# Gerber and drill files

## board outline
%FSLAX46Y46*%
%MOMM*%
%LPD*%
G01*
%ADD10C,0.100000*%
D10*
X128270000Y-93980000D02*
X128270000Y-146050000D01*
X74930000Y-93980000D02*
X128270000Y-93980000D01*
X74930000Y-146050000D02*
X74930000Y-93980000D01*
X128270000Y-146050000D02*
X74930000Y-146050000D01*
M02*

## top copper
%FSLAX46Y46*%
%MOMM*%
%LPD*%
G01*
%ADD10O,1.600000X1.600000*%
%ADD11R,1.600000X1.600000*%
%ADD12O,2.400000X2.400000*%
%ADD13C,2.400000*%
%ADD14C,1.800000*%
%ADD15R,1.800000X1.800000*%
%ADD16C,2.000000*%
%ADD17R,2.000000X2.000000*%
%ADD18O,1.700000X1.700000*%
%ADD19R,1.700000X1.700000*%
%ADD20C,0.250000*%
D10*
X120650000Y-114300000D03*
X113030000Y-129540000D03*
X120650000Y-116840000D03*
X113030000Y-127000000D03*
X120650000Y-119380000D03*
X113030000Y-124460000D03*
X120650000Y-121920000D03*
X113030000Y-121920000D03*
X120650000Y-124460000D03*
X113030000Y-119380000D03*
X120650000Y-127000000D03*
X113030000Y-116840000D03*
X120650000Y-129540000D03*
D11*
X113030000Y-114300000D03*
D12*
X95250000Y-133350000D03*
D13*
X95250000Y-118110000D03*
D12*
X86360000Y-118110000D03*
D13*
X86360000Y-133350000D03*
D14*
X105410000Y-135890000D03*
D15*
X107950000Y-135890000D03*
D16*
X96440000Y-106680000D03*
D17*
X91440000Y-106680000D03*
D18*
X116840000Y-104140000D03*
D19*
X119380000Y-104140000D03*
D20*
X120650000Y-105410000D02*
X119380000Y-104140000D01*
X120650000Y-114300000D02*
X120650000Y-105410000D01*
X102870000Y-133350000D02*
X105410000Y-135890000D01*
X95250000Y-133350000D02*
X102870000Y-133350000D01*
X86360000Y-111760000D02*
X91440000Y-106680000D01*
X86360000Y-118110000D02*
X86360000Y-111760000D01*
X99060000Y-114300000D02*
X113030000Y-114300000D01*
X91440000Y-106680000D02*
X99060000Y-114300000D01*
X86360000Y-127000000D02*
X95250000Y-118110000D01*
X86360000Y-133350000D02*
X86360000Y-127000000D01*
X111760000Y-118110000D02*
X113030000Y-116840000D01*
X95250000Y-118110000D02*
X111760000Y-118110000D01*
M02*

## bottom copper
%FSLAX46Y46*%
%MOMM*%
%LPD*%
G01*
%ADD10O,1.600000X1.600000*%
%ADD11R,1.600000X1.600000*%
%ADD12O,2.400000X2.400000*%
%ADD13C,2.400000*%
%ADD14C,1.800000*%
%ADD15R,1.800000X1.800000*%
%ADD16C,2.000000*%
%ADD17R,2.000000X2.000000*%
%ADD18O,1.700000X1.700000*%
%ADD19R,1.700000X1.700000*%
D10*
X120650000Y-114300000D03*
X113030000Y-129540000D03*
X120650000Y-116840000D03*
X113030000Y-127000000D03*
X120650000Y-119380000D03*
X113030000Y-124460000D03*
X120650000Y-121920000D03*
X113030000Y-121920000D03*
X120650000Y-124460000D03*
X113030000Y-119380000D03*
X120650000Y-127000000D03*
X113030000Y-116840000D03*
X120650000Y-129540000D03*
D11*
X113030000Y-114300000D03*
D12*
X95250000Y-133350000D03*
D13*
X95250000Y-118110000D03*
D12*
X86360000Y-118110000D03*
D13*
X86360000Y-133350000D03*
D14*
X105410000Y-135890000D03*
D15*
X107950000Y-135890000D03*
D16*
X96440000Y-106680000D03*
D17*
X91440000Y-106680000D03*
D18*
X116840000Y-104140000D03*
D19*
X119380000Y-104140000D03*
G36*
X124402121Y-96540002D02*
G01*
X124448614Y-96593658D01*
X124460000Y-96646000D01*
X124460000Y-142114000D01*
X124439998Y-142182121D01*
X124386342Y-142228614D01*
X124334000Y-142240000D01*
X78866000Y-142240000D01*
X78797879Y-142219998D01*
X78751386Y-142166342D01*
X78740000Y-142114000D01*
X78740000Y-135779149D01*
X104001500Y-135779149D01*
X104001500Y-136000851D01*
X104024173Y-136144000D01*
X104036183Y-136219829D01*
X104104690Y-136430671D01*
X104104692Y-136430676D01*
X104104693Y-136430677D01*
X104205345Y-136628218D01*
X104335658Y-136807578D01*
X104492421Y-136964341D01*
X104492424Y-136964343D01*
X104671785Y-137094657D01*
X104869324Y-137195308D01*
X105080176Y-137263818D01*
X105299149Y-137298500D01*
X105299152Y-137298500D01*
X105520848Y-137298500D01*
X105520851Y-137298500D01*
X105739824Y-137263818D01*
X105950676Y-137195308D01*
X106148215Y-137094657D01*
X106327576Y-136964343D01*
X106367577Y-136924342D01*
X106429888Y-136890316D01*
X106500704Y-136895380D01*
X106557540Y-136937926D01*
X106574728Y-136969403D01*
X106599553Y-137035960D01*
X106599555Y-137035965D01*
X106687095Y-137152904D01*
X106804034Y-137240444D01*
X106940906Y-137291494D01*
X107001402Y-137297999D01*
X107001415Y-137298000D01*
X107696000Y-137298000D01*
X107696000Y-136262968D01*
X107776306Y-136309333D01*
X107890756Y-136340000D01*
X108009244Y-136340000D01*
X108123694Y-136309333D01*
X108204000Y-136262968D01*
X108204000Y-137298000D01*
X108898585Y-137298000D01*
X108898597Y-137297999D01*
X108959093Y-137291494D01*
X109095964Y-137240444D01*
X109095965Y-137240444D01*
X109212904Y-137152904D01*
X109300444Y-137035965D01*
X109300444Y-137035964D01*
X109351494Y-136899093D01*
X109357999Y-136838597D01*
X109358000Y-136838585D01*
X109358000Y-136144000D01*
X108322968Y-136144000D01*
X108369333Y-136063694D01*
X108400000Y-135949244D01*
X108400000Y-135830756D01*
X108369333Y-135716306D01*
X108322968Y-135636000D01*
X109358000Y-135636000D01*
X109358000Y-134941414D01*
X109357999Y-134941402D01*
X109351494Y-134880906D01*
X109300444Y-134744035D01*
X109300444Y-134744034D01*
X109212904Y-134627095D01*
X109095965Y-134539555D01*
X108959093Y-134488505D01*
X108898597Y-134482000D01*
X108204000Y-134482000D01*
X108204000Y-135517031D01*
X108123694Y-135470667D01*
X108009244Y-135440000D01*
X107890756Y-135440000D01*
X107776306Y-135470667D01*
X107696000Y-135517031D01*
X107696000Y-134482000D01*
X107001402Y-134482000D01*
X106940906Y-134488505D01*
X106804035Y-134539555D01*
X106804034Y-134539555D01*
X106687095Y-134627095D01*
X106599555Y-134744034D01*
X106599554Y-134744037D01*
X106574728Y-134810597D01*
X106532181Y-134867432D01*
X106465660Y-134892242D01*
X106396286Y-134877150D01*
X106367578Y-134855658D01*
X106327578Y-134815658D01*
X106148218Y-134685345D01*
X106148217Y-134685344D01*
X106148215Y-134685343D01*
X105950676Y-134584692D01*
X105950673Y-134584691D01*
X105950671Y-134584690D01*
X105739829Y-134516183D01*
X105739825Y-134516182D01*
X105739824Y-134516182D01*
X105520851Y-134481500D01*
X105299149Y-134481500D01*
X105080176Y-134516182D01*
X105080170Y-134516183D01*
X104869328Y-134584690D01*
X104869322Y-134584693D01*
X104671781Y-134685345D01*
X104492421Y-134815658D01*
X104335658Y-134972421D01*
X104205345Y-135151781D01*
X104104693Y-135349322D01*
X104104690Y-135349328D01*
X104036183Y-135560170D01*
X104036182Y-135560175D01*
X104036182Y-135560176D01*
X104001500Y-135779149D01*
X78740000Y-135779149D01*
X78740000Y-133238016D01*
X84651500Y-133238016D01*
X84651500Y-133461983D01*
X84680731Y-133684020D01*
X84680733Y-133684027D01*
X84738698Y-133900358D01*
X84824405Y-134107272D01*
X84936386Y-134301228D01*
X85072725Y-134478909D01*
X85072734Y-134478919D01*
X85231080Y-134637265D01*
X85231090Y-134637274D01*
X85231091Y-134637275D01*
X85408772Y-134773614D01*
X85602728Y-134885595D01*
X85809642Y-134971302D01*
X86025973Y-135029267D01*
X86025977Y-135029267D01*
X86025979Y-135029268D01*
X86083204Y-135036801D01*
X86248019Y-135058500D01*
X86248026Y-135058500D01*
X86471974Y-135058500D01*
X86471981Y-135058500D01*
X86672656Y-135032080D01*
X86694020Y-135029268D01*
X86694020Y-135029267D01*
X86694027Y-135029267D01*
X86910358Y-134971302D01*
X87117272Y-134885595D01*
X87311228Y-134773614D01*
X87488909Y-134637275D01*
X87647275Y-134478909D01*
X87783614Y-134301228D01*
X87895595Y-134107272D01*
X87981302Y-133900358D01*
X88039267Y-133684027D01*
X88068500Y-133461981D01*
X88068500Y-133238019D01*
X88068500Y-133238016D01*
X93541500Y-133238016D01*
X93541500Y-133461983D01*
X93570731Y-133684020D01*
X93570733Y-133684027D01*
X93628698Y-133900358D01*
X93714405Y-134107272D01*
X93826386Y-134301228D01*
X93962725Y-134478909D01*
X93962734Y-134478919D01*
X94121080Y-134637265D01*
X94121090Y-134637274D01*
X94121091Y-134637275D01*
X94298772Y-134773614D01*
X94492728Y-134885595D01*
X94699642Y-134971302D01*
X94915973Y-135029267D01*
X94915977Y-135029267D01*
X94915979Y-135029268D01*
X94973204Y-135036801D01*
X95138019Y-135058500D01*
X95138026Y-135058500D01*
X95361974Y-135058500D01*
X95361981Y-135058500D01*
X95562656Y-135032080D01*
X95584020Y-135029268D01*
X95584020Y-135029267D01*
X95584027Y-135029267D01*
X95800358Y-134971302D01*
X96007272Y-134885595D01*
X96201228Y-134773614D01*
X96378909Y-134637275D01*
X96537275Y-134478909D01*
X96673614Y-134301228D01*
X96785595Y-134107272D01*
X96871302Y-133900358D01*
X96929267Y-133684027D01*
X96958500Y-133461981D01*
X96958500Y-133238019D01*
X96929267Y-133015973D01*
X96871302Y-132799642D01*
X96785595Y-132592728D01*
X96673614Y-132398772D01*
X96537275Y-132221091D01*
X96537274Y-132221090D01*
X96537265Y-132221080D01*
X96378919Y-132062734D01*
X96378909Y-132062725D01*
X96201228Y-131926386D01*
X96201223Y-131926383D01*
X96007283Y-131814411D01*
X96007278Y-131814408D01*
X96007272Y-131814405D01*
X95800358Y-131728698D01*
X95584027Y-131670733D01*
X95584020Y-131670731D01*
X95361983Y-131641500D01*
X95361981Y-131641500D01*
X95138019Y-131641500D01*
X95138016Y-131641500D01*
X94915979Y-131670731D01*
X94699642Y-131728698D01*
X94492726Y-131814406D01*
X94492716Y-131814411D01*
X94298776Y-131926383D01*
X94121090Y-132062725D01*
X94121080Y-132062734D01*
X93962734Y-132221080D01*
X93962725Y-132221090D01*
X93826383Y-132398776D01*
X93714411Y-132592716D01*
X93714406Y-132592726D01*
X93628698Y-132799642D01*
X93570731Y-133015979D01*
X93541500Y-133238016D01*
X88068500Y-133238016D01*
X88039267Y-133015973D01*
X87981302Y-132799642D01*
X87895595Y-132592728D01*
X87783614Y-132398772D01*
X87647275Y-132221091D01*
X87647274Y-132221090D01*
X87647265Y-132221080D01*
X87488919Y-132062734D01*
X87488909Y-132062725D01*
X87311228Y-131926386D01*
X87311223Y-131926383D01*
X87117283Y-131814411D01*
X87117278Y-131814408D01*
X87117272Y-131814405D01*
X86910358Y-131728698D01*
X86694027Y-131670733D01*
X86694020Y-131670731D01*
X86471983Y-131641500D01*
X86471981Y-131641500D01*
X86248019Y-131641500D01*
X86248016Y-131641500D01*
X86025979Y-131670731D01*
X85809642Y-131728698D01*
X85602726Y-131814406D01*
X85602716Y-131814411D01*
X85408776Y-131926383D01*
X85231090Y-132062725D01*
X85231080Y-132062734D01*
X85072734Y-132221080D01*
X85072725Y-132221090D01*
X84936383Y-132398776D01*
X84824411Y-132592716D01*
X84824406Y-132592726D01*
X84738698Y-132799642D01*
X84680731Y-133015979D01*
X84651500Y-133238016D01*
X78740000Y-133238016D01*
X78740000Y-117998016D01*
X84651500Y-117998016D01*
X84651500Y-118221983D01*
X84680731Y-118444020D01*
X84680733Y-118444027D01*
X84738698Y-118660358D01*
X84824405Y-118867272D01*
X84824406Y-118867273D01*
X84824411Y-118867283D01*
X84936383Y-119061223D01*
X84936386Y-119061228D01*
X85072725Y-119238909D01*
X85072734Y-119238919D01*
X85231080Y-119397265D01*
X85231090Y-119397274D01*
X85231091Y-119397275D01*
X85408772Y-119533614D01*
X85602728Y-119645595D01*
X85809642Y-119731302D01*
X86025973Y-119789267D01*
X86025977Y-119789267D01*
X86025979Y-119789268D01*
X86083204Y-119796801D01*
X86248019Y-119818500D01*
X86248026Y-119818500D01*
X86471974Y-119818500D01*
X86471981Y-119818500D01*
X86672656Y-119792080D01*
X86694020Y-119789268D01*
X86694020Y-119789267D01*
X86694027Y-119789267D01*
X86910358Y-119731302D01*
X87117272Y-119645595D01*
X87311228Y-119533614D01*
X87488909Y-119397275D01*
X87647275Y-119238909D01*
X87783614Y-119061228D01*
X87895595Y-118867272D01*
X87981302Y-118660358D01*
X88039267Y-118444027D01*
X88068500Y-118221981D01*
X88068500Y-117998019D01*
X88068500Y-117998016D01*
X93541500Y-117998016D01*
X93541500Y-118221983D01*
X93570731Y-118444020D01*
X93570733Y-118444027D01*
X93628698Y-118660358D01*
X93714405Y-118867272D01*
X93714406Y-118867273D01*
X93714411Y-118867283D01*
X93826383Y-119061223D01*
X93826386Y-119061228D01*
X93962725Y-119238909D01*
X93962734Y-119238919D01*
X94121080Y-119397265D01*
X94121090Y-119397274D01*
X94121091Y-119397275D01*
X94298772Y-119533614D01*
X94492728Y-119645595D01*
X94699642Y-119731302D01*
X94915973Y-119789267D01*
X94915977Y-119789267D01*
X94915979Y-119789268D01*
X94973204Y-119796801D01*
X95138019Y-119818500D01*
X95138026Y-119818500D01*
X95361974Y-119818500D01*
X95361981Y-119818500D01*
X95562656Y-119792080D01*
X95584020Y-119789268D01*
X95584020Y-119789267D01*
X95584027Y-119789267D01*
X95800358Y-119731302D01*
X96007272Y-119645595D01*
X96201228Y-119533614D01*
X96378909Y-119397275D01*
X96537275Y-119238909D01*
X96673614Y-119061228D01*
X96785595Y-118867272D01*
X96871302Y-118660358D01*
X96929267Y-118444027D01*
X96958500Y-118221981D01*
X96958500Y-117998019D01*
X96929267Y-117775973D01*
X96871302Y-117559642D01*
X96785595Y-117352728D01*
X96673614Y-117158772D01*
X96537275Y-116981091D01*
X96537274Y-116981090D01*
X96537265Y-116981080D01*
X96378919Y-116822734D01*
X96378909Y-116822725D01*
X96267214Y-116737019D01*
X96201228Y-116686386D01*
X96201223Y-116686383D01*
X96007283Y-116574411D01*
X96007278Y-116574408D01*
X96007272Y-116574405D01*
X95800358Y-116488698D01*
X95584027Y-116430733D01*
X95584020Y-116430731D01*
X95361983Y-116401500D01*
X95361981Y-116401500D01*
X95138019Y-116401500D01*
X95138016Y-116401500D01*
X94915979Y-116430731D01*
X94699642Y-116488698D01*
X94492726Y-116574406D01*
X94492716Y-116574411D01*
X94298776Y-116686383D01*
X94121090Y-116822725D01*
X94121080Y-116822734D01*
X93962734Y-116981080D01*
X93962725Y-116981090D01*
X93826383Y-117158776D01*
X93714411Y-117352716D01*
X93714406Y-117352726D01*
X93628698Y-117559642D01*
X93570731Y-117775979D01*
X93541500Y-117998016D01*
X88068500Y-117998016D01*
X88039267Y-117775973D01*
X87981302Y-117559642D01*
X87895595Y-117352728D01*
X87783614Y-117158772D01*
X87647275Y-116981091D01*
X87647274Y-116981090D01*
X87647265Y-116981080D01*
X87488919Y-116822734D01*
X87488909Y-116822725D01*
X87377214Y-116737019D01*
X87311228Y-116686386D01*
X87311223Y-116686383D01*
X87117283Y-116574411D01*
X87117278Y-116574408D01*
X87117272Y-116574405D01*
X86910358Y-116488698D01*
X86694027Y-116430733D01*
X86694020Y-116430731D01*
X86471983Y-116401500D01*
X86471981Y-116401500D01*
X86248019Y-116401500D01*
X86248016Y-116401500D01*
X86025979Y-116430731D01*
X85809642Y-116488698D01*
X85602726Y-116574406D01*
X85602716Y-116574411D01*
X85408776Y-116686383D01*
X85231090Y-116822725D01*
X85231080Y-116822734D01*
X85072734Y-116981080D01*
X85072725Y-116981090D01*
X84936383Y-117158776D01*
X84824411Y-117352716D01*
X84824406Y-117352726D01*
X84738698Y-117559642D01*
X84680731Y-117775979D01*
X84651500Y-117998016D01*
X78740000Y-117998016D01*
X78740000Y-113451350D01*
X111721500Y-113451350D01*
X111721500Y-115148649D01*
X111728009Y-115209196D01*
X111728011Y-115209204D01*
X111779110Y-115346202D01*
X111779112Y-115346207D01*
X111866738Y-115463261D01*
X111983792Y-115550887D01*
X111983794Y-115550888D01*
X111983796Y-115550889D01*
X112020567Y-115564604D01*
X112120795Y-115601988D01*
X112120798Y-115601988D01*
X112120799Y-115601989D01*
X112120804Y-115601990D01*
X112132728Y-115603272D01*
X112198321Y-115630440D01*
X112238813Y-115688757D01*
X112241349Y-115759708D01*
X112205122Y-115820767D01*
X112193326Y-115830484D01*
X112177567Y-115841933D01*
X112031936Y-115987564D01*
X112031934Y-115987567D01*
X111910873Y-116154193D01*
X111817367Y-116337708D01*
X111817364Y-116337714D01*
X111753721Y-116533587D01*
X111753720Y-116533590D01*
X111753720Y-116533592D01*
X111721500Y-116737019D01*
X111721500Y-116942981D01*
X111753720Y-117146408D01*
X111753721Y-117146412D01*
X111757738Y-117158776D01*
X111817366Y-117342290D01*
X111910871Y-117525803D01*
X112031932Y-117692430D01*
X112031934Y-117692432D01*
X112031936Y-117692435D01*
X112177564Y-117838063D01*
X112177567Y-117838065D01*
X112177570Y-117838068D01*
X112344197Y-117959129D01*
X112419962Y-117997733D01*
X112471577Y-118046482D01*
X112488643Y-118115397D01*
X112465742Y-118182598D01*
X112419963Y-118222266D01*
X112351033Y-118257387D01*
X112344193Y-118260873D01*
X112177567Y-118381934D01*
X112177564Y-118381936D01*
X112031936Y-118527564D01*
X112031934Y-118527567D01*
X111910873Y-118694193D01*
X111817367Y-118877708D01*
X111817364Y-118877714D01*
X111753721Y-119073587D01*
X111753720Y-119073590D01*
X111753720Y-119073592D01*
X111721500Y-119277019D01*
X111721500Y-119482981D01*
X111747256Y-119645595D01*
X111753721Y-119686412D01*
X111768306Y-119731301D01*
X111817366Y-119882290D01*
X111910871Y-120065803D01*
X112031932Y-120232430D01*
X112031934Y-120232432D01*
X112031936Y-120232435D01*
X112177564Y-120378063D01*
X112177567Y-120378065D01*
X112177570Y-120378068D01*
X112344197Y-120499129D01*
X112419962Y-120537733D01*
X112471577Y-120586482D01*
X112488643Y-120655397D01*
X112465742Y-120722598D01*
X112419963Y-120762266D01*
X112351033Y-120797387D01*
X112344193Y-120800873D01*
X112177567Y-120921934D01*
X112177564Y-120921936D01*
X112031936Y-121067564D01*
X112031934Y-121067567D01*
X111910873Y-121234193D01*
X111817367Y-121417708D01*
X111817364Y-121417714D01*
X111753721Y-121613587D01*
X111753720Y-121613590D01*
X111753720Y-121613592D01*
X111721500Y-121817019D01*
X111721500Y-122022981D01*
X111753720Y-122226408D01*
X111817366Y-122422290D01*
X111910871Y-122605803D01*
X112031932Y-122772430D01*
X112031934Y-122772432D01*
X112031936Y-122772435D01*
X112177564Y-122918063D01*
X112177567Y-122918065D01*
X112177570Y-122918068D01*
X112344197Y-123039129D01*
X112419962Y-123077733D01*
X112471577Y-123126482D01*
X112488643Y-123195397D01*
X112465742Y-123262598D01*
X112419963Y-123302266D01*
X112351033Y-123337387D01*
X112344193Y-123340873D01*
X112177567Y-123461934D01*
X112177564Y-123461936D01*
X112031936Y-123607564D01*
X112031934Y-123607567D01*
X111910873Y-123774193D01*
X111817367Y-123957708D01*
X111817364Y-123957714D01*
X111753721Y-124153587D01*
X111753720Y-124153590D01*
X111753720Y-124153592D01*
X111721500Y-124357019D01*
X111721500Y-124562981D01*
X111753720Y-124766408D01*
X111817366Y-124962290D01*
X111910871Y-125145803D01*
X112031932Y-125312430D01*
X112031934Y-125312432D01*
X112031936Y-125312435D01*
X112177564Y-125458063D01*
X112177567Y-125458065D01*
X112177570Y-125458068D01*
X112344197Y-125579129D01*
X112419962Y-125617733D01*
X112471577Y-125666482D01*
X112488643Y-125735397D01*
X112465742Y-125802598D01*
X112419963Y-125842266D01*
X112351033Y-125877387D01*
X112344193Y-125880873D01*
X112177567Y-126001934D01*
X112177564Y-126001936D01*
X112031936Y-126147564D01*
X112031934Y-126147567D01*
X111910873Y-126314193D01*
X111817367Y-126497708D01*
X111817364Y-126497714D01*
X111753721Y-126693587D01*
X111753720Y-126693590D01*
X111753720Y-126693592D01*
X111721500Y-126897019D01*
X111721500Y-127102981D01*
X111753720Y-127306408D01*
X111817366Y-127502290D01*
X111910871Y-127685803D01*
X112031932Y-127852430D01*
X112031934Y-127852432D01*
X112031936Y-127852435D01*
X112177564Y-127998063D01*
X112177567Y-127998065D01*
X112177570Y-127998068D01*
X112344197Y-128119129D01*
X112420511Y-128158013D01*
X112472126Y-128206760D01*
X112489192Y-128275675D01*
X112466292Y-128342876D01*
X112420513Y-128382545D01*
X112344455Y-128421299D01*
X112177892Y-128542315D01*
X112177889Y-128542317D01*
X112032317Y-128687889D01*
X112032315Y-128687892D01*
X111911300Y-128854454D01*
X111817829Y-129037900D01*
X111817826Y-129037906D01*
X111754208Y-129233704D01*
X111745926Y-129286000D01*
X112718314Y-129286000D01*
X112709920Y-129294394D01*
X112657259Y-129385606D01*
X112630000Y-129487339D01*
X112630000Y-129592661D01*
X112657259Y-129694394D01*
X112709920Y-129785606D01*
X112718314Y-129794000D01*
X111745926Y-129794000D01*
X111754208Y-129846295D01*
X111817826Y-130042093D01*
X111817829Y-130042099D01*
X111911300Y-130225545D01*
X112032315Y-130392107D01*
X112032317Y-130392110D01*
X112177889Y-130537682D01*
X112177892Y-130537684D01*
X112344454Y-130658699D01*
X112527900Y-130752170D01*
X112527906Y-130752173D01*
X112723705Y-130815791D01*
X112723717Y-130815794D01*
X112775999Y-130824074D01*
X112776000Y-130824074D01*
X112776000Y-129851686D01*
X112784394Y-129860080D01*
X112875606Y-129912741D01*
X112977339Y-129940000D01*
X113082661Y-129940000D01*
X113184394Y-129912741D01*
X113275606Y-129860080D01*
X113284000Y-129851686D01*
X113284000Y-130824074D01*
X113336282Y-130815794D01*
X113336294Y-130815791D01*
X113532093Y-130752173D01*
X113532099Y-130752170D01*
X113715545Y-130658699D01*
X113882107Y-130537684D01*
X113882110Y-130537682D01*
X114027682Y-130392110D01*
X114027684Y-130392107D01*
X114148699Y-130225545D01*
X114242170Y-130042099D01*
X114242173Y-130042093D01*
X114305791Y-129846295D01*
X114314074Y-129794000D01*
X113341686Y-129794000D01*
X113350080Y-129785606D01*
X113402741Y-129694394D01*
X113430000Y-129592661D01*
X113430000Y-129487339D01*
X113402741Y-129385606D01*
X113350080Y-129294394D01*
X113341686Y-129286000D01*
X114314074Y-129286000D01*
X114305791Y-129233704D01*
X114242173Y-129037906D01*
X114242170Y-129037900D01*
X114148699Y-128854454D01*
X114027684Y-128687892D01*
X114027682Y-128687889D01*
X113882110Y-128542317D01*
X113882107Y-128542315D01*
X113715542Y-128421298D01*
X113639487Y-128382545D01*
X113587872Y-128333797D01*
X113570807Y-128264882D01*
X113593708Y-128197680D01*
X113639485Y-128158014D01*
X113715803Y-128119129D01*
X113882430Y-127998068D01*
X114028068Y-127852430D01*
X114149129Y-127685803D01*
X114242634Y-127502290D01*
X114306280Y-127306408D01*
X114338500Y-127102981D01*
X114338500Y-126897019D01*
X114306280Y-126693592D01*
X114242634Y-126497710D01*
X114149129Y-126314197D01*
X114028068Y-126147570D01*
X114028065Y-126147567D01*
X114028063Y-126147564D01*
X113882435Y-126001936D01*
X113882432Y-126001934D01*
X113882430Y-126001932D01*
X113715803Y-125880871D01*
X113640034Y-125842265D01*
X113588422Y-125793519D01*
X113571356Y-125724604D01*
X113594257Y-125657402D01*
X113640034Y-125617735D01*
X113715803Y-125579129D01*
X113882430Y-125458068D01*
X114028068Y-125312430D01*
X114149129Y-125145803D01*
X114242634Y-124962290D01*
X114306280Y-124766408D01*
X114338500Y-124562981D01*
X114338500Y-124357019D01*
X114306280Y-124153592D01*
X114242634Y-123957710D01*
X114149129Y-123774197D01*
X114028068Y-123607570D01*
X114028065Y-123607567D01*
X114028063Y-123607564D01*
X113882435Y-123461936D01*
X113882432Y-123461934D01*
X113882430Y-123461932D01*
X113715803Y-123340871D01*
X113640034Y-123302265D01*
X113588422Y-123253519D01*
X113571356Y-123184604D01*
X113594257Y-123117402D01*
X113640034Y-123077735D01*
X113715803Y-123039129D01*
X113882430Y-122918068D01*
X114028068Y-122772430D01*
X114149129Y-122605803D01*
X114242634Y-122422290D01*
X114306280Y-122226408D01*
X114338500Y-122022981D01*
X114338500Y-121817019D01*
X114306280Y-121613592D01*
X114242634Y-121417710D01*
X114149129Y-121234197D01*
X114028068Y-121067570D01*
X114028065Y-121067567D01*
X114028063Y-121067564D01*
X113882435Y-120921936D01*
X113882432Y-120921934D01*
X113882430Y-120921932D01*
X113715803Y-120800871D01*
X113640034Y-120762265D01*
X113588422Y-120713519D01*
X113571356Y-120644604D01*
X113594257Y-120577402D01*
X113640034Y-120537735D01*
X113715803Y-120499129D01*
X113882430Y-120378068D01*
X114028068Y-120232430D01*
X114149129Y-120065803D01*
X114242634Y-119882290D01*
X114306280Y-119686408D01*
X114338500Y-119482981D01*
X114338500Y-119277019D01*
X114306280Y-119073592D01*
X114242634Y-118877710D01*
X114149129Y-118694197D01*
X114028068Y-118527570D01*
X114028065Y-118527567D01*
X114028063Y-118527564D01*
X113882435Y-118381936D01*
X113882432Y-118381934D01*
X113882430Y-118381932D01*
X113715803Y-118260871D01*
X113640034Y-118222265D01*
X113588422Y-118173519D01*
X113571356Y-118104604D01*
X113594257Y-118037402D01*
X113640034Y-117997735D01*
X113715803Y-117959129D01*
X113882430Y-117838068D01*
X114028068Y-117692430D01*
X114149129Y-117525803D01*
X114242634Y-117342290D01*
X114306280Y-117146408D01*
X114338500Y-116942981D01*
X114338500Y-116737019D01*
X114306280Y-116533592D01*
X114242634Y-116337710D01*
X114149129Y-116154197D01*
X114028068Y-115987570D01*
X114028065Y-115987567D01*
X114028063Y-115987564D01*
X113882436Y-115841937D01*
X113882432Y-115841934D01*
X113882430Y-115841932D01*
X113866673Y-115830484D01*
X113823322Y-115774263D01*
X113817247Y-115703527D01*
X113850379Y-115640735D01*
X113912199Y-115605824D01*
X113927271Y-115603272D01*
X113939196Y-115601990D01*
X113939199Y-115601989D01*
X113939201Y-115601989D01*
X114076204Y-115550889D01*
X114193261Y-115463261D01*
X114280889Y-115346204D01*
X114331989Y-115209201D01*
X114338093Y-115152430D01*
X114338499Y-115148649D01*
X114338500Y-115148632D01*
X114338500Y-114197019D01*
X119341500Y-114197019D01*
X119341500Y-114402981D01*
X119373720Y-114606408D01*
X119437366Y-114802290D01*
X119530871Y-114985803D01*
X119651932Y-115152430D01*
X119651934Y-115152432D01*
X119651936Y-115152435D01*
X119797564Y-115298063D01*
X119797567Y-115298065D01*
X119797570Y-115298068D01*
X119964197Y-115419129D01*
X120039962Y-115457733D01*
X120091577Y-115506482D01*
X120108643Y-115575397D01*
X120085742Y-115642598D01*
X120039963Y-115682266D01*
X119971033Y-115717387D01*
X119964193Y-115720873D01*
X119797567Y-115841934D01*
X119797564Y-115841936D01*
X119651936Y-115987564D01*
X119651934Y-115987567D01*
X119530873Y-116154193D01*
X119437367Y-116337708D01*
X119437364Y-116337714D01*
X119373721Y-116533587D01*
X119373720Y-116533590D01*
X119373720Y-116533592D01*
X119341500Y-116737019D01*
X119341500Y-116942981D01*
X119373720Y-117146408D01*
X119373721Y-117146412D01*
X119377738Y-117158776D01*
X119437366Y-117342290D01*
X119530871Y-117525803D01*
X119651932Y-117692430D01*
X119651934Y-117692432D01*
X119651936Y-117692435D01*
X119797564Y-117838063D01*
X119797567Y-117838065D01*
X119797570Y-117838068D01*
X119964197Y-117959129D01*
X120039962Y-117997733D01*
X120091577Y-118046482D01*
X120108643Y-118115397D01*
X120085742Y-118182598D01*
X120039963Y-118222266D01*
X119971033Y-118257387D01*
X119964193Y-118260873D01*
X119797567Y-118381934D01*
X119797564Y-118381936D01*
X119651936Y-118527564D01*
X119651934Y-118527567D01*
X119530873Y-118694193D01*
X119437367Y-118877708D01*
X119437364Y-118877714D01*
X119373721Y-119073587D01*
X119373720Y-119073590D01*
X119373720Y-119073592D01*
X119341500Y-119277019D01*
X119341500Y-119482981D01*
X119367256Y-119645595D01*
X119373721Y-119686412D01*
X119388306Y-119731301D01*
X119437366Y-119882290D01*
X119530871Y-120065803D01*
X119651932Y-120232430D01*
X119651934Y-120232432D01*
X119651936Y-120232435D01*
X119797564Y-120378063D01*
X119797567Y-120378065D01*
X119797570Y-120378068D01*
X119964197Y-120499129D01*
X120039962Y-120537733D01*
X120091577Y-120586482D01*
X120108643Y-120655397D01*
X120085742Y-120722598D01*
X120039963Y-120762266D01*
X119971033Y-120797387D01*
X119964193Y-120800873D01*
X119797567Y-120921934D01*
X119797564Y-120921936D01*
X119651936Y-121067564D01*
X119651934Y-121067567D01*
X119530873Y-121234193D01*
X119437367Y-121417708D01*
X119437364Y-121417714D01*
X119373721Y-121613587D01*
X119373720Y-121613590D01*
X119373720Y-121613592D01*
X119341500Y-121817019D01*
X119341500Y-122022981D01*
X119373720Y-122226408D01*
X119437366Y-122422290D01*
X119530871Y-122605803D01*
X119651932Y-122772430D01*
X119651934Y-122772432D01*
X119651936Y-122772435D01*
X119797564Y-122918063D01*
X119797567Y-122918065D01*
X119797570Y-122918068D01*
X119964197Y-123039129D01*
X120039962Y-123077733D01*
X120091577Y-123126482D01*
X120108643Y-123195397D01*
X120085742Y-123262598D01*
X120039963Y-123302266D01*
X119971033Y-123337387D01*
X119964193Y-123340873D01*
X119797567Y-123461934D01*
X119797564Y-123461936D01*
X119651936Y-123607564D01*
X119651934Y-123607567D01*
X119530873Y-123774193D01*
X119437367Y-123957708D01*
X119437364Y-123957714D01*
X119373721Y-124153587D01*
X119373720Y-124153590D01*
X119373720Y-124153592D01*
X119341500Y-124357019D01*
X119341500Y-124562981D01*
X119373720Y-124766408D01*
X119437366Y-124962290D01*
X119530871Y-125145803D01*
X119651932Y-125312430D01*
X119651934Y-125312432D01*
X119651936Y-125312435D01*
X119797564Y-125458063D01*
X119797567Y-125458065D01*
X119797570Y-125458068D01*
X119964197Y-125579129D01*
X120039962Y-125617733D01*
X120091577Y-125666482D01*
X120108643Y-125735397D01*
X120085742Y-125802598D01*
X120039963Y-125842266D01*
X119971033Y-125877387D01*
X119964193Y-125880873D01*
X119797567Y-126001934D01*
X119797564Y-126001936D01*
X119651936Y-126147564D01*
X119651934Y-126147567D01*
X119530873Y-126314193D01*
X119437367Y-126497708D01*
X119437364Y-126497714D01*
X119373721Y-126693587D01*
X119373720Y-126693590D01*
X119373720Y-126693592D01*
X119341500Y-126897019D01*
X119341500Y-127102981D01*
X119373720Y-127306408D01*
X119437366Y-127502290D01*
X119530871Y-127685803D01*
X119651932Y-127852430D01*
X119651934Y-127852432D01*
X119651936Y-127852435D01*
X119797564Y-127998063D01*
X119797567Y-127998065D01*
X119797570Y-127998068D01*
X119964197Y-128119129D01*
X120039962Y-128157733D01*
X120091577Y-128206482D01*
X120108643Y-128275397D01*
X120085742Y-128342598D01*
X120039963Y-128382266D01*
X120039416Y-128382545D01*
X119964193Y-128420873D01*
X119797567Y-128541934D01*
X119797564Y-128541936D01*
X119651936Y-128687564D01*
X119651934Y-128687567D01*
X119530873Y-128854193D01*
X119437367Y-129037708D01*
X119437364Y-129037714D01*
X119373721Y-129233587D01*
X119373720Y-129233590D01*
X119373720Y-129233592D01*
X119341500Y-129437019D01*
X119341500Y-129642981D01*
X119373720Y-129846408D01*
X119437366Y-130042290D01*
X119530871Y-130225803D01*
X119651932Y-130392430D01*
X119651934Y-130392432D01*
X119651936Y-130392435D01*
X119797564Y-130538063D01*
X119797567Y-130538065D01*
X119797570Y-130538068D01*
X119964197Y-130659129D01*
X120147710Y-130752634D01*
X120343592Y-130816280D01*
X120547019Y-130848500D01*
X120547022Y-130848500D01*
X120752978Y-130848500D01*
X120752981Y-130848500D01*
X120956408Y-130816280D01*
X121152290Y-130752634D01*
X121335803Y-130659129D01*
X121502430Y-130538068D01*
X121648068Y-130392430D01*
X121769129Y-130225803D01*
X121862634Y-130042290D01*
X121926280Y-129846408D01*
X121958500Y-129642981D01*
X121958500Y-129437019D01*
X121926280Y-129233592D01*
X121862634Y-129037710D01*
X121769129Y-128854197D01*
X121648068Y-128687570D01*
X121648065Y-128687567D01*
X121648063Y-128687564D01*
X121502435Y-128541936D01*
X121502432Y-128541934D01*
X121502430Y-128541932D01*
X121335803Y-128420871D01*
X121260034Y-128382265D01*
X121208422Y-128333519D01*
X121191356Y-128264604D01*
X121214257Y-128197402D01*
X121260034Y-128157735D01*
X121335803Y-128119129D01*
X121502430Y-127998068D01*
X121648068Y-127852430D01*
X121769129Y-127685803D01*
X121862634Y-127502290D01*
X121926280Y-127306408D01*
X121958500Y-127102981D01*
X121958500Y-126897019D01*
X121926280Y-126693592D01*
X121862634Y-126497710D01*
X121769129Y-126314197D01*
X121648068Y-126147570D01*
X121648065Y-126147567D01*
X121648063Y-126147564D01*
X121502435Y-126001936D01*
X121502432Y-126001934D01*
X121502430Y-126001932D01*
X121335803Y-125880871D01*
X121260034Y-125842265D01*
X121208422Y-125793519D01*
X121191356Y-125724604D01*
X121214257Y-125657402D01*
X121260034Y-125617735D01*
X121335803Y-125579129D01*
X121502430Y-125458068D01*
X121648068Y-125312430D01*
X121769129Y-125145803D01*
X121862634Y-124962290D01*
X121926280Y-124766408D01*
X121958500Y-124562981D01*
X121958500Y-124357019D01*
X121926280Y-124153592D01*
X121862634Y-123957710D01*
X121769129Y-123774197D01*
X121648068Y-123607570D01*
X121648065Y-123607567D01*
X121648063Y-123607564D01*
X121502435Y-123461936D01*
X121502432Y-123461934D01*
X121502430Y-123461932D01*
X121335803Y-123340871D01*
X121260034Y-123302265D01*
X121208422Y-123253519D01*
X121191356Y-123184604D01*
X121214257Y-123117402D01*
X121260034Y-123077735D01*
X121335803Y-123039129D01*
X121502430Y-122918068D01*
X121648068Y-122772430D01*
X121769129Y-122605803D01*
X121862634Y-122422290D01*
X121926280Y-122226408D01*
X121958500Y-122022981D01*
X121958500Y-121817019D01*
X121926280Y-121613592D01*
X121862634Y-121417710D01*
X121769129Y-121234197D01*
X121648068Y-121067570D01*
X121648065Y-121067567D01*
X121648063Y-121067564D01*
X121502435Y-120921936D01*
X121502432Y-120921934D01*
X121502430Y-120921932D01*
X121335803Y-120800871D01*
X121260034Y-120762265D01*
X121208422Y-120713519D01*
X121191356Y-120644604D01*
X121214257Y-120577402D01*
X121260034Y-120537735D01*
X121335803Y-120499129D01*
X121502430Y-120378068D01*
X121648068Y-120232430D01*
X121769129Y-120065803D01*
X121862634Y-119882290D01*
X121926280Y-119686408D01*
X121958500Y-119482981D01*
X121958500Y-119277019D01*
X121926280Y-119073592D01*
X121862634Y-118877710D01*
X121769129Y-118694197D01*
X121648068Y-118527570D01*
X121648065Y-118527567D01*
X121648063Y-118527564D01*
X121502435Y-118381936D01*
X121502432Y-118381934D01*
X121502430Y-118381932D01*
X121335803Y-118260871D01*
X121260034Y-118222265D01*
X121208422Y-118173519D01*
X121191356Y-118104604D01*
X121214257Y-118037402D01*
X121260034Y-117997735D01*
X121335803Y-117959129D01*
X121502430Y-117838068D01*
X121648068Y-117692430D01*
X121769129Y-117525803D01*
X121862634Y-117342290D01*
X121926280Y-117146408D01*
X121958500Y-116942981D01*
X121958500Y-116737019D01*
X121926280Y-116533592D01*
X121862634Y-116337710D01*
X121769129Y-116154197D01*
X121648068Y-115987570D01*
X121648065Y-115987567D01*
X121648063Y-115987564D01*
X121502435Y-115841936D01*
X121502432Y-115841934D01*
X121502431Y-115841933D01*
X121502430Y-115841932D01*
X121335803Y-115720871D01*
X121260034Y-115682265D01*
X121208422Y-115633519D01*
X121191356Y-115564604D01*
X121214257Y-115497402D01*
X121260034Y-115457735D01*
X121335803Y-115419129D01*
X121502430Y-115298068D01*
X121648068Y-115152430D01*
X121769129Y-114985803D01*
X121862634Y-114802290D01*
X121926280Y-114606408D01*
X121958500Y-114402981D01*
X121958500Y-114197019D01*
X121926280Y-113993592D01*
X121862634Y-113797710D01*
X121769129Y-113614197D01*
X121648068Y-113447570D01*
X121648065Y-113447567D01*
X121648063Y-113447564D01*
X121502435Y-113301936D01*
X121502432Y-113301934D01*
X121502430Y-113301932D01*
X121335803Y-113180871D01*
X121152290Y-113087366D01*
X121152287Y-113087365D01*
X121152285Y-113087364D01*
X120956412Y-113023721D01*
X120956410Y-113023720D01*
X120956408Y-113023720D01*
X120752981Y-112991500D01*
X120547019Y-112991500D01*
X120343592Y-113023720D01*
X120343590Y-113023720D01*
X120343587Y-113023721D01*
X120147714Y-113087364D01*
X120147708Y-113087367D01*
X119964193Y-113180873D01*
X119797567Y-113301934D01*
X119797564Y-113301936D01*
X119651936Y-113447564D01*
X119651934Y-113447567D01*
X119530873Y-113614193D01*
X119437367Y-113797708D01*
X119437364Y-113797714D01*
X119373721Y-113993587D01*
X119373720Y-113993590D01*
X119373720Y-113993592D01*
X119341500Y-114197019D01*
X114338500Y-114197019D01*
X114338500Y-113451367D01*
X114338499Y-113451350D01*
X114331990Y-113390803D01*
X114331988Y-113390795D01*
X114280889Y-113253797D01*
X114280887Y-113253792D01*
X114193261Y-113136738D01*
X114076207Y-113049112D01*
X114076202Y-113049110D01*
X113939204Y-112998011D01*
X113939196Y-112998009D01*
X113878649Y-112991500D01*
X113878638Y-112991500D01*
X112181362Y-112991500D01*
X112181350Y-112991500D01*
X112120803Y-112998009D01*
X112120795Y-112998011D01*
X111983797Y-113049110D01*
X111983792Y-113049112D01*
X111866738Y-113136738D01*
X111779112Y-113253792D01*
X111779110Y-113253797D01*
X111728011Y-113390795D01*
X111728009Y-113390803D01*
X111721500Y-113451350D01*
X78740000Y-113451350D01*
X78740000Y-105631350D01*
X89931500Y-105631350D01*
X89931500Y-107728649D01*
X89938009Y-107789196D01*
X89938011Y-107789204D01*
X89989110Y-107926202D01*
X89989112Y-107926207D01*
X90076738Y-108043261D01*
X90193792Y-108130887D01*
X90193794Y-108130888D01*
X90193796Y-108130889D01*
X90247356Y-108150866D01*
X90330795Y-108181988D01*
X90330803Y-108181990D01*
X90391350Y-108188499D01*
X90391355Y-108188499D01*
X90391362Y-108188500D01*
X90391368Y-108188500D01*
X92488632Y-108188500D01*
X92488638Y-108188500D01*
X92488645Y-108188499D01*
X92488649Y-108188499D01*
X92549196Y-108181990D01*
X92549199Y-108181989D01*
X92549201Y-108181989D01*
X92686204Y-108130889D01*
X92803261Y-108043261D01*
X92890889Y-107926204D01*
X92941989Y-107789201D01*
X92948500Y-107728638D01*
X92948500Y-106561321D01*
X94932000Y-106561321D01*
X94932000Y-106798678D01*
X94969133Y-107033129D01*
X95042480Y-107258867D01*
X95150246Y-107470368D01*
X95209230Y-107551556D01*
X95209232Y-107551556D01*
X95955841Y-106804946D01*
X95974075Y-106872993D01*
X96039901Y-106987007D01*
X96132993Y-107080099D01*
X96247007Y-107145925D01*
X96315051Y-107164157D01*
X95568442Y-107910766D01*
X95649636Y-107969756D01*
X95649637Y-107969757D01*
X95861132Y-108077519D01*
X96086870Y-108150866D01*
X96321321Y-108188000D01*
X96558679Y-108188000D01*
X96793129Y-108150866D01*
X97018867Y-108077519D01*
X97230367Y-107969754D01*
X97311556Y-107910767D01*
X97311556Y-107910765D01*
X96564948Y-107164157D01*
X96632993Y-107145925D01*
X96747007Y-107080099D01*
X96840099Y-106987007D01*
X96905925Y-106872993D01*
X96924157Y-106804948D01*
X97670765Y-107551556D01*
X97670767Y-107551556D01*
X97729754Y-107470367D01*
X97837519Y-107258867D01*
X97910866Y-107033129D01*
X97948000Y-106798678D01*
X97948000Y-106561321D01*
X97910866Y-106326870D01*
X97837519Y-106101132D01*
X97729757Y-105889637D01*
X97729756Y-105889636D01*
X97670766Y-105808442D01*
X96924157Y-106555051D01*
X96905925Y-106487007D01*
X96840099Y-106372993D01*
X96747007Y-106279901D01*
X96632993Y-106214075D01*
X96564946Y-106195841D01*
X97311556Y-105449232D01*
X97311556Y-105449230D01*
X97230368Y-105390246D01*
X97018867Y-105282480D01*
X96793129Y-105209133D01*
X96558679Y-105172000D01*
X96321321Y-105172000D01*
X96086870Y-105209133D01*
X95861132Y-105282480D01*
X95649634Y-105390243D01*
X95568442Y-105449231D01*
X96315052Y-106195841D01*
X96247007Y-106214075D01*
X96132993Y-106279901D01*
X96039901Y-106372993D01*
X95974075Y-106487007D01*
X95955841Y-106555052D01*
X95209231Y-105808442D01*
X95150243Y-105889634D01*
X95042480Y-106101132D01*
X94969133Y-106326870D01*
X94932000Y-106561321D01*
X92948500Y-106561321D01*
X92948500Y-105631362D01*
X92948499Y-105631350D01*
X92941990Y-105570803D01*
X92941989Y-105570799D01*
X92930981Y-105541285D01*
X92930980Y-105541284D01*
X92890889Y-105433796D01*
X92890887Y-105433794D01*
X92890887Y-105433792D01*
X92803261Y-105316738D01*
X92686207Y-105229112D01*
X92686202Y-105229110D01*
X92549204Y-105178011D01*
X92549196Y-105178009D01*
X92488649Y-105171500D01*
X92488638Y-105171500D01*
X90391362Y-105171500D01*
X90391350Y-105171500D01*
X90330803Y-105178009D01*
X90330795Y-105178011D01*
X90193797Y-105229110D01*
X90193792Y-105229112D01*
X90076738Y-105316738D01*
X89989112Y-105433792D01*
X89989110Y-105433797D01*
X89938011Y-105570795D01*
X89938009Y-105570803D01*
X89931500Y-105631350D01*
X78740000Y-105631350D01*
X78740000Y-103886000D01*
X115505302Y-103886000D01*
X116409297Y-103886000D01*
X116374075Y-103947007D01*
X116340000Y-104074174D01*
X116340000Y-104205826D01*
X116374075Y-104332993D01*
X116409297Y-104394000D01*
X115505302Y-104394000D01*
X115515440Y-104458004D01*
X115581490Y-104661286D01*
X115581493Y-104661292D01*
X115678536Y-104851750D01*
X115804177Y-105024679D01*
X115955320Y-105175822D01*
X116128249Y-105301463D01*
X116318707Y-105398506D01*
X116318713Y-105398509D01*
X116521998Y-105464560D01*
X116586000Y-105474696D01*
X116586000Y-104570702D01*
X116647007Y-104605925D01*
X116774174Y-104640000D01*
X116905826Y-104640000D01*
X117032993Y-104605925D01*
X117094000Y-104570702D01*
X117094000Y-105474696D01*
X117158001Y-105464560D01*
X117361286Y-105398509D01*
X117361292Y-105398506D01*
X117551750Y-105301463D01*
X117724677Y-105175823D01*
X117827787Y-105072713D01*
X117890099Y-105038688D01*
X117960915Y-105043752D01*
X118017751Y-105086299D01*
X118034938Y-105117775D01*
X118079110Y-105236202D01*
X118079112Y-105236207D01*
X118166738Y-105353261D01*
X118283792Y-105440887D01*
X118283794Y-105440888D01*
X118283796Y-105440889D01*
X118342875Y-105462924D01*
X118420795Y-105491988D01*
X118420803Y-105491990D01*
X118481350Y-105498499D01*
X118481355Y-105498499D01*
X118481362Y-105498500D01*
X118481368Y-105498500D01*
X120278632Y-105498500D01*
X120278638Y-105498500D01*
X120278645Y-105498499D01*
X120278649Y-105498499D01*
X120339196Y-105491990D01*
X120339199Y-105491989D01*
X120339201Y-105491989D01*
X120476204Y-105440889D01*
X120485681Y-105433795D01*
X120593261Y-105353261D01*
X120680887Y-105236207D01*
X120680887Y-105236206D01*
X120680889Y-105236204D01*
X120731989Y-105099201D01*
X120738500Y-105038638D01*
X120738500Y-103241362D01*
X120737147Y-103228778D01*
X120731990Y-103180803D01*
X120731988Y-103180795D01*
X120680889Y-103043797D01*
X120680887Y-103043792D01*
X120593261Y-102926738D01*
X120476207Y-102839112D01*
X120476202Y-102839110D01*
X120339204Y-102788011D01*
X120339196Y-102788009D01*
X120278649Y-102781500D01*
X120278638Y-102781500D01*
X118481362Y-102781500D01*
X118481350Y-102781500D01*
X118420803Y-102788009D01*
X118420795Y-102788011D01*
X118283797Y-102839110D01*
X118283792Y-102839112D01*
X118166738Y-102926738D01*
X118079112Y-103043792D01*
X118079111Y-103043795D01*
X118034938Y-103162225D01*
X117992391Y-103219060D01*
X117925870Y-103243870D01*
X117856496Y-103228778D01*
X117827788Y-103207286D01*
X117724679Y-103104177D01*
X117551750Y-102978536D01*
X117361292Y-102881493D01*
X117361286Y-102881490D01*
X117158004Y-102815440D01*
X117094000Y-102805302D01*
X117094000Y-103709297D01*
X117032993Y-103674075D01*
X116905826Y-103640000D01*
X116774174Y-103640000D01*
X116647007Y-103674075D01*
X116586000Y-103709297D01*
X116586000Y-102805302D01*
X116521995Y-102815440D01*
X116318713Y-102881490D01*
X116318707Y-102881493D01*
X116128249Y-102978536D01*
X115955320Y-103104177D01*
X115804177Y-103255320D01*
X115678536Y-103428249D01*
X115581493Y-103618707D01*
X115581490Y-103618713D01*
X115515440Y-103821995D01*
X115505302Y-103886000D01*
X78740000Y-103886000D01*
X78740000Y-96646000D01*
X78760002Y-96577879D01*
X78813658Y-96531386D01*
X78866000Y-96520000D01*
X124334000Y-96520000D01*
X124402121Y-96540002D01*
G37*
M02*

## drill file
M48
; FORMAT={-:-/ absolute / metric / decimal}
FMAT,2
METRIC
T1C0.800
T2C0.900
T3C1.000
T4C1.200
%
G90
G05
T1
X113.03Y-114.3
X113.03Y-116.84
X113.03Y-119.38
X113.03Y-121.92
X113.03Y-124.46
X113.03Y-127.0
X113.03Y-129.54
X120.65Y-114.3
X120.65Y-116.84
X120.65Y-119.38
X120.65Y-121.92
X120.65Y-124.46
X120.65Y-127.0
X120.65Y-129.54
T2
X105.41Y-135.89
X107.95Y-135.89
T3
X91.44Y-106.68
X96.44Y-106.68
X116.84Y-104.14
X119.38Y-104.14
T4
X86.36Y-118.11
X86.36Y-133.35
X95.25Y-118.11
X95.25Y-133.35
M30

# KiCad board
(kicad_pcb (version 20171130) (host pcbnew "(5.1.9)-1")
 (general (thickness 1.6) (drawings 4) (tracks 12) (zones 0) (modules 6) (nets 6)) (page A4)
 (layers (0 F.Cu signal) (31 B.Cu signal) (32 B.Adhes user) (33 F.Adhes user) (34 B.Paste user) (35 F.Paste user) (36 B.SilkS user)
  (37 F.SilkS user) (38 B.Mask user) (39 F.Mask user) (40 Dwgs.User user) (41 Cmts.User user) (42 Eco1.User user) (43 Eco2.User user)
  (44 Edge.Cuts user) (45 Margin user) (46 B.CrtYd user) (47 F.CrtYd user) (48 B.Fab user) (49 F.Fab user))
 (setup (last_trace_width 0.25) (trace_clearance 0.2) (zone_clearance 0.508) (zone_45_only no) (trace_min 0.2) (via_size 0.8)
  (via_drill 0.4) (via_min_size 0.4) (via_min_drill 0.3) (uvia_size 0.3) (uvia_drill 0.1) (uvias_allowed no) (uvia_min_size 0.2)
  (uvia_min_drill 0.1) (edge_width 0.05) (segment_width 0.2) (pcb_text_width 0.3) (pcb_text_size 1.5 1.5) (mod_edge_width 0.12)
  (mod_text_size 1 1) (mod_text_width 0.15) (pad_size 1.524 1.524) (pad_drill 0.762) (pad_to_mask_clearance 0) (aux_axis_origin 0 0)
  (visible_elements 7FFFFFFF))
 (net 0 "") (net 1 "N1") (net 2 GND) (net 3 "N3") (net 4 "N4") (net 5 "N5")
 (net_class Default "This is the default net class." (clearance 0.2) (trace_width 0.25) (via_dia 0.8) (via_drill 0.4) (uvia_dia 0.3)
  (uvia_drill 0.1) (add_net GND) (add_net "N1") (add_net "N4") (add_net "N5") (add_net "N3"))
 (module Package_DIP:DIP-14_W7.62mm (layer F.Cu) (at 113.03 114.3)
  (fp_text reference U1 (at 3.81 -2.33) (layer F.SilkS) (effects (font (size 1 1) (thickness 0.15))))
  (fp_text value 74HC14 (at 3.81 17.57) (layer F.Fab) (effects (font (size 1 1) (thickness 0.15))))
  (pad 14 thru_hole oval (at 7.62 0) (size 1.6 1.6) (drill 0.8) (layers *.Cu *.Mask) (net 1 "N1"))
  (pad 7 thru_hole oval (at 0 15.24) (size 1.6 1.6) (drill 0.8) (layers *.Cu *.Mask) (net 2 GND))
  (pad 13 thru_hole oval (at 7.62 2.54) (size 1.6 1.6) (drill 0.8) (layers *.Cu *.Mask))
  (pad 6 thru_hole oval (at 0 12.7) (size 1.6 1.6) (drill 0.8) (layers *.Cu *.Mask))
  (pad 12 thru_hole oval (at 7.62 5.08) (size 1.6 1.6) (drill 0.8) (layers *.Cu *.Mask))
  (pad 5 thru_hole oval (at 0 10.16) (size 1.6 1.6) (drill 0.8) (layers *.Cu *.Mask))
  (pad 11 thru_hole oval (at 7.62 7.62) (size 1.6 1.6) (drill 0.8) (layers *.Cu *.Mask))
  (pad 4 thru_hole oval (at 0 7.62) (size 1.6 1.6) (drill 0.8) (layers *.Cu *.Mask))
  (pad 10 thru_hole oval (at 7.62 10.16) (size 1.6 1.6) (drill 0.8) (layers *.Cu *.Mask))
  (pad 3 thru_hole oval (at 0 5.08) (size 1.6 1.6) (drill 0.8) (layers *.Cu *.Mask))
  (pad 9 thru_hole oval (at 7.62 12.7) (size 1.6 1.6) (drill 0.8) (layers *.Cu *.Mask))
  (pad 2 thru_hole oval (at 0 2.54) (size 1.6 1.6) (drill 0.8) (layers *.Cu *.Mask) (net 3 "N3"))
  (pad 8 thru_hole oval (at 7.62 15.24) (size 1.6 1.6) (drill 0.8) (layers *.Cu *.Mask))
  (pad 1 thru_hole rect (at 0 0) (size 1.6 1.6) (drill 0.8) (layers *.Cu *.Mask) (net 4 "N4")))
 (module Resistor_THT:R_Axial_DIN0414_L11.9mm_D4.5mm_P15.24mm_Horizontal (layer F.Cu) (at 95.25 118.11 270)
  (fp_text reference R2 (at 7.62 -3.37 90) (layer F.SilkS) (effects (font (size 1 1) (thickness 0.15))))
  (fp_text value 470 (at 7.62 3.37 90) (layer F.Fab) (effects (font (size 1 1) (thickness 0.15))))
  (pad 2 thru_hole oval (at 15.24 0 270) (size 2.4 2.4) (drill 1.2) (layers *.Cu *.Mask) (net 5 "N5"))
  (pad 1 thru_hole circle (at 0 0 270) (size 2.4 2.4) (drill 1.2) (layers *.Cu *.Mask) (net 3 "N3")))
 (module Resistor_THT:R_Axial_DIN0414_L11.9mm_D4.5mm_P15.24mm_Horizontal (layer F.Cu) (at 86.36 133.35 90)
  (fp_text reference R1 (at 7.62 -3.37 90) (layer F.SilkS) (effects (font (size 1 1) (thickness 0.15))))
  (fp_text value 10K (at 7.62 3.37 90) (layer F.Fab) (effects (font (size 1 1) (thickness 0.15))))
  (pad 2 thru_hole oval (at 15.24 0 90) (size 2.4 2.4) (drill 1.2) (layers *.Cu *.Mask) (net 4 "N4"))
  (pad 1 thru_hole circle (at 0 0 90) (size 2.4 2.4) (drill 1.2) (layers *.Cu *.Mask) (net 3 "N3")))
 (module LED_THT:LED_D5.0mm (layer F.Cu) (at 107.95 135.89 180)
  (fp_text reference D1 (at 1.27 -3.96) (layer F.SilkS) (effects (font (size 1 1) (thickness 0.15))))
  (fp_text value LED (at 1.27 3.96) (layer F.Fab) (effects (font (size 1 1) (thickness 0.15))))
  (pad 2 thru_hole circle (at 2.54 0 180) (size 1.8 1.8) (drill 0.9) (layers *.Cu *.Mask) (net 5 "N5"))
  (pad 1 thru_hole rect (at 0 0 180) (size 1.8 1.8) (drill 0.9) (layers *.Cu *.Mask) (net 2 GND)))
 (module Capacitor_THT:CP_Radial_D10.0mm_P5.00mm (layer F.Cu) (at 91.44 106.68)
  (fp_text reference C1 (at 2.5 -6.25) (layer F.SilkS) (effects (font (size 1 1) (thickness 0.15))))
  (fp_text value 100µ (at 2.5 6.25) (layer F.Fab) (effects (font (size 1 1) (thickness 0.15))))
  (pad 2 thru_hole circle (at 5 0) (size 2 2) (drill 1) (layers *.Cu *.Mask) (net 2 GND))
  (pad 1 thru_hole rect (at 0 0) (size 2 2) (drill 1) (layers *.Cu *.Mask) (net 4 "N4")))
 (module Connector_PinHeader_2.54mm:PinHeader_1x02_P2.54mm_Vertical (layer F.Cu) (at 119.38 104.14 270)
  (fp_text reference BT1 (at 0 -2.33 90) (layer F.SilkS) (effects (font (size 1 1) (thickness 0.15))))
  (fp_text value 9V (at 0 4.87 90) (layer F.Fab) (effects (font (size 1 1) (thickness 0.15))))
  (pad 2 thru_hole oval (at 0 2.54 270) (size 1.7 1.7) (drill 1) (layers *.Cu *.Mask) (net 2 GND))
  (pad 1 thru_hole rect (at 0 0 270) (size 1.7 1.7) (drill 1) (layers *.Cu *.Mask) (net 1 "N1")))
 (gr_line (start 128.27 93.98) (end 128.27 146.05) (layer Edge.Cuts) (width 0.1))
 (gr_line (start 74.93 93.98) (end 128.27 93.98) (layer Edge.Cuts) (width 0.1))
 (gr_line (start 74.93 146.05) (end 74.93 93.98) (layer Edge.Cuts) (width 0.1))
 (gr_line (start 128.27 146.05) (end 74.93 146.05) (layer Edge.Cuts) (width 0.1))
 (segment (start 120.65 105.41) (end 119.38 104.14) (width 0.25) (layer F.Cu) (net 1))
 (segment (start 120.65 114.3) (end 120.65 105.41) (width 0.25) (layer F.Cu) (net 1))
 (segment (start 102.87 133.35) (end 105.41 135.89) (width 0.25) (layer F.Cu) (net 5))
 (segment (start 95.25 133.35) (end 102.87 133.35) (width 0.25) (layer F.Cu) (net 5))
 (segment (start 86.36 111.76) (end 91.44 106.68) (width 0.25) (layer F.Cu) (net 4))
 (segment (start 86.36 118.11) (end 86.36 111.76) (width 0.25) (layer F.Cu) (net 4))
 (segment (start 99.06 114.3) (end 113.03 114.3) (width 0.25) (layer F.Cu) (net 4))
 (segment (start 91.44 106.68) (end 99.06 114.3) (width 0.25) (layer F.Cu) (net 4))
 (segment (start 86.36 127) (end 95.25 118.11) (width 0.25) (layer F.Cu) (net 3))
 (segment (start 86.36 133.35) (end 86.36 127) (width 0.25) (layer F.Cu) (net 3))
 (segment (start 111.76 118.11) (end 113.03 116.84) (width 0.25) (layer F.Cu) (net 3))
 (segment (start 95.25 118.11) (end 111.76 118.11) (width 0.25) (layer F.Cu) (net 3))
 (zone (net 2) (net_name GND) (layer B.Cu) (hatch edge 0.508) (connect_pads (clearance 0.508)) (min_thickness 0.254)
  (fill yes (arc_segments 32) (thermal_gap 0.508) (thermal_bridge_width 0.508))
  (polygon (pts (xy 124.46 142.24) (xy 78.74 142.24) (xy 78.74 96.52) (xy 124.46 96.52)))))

